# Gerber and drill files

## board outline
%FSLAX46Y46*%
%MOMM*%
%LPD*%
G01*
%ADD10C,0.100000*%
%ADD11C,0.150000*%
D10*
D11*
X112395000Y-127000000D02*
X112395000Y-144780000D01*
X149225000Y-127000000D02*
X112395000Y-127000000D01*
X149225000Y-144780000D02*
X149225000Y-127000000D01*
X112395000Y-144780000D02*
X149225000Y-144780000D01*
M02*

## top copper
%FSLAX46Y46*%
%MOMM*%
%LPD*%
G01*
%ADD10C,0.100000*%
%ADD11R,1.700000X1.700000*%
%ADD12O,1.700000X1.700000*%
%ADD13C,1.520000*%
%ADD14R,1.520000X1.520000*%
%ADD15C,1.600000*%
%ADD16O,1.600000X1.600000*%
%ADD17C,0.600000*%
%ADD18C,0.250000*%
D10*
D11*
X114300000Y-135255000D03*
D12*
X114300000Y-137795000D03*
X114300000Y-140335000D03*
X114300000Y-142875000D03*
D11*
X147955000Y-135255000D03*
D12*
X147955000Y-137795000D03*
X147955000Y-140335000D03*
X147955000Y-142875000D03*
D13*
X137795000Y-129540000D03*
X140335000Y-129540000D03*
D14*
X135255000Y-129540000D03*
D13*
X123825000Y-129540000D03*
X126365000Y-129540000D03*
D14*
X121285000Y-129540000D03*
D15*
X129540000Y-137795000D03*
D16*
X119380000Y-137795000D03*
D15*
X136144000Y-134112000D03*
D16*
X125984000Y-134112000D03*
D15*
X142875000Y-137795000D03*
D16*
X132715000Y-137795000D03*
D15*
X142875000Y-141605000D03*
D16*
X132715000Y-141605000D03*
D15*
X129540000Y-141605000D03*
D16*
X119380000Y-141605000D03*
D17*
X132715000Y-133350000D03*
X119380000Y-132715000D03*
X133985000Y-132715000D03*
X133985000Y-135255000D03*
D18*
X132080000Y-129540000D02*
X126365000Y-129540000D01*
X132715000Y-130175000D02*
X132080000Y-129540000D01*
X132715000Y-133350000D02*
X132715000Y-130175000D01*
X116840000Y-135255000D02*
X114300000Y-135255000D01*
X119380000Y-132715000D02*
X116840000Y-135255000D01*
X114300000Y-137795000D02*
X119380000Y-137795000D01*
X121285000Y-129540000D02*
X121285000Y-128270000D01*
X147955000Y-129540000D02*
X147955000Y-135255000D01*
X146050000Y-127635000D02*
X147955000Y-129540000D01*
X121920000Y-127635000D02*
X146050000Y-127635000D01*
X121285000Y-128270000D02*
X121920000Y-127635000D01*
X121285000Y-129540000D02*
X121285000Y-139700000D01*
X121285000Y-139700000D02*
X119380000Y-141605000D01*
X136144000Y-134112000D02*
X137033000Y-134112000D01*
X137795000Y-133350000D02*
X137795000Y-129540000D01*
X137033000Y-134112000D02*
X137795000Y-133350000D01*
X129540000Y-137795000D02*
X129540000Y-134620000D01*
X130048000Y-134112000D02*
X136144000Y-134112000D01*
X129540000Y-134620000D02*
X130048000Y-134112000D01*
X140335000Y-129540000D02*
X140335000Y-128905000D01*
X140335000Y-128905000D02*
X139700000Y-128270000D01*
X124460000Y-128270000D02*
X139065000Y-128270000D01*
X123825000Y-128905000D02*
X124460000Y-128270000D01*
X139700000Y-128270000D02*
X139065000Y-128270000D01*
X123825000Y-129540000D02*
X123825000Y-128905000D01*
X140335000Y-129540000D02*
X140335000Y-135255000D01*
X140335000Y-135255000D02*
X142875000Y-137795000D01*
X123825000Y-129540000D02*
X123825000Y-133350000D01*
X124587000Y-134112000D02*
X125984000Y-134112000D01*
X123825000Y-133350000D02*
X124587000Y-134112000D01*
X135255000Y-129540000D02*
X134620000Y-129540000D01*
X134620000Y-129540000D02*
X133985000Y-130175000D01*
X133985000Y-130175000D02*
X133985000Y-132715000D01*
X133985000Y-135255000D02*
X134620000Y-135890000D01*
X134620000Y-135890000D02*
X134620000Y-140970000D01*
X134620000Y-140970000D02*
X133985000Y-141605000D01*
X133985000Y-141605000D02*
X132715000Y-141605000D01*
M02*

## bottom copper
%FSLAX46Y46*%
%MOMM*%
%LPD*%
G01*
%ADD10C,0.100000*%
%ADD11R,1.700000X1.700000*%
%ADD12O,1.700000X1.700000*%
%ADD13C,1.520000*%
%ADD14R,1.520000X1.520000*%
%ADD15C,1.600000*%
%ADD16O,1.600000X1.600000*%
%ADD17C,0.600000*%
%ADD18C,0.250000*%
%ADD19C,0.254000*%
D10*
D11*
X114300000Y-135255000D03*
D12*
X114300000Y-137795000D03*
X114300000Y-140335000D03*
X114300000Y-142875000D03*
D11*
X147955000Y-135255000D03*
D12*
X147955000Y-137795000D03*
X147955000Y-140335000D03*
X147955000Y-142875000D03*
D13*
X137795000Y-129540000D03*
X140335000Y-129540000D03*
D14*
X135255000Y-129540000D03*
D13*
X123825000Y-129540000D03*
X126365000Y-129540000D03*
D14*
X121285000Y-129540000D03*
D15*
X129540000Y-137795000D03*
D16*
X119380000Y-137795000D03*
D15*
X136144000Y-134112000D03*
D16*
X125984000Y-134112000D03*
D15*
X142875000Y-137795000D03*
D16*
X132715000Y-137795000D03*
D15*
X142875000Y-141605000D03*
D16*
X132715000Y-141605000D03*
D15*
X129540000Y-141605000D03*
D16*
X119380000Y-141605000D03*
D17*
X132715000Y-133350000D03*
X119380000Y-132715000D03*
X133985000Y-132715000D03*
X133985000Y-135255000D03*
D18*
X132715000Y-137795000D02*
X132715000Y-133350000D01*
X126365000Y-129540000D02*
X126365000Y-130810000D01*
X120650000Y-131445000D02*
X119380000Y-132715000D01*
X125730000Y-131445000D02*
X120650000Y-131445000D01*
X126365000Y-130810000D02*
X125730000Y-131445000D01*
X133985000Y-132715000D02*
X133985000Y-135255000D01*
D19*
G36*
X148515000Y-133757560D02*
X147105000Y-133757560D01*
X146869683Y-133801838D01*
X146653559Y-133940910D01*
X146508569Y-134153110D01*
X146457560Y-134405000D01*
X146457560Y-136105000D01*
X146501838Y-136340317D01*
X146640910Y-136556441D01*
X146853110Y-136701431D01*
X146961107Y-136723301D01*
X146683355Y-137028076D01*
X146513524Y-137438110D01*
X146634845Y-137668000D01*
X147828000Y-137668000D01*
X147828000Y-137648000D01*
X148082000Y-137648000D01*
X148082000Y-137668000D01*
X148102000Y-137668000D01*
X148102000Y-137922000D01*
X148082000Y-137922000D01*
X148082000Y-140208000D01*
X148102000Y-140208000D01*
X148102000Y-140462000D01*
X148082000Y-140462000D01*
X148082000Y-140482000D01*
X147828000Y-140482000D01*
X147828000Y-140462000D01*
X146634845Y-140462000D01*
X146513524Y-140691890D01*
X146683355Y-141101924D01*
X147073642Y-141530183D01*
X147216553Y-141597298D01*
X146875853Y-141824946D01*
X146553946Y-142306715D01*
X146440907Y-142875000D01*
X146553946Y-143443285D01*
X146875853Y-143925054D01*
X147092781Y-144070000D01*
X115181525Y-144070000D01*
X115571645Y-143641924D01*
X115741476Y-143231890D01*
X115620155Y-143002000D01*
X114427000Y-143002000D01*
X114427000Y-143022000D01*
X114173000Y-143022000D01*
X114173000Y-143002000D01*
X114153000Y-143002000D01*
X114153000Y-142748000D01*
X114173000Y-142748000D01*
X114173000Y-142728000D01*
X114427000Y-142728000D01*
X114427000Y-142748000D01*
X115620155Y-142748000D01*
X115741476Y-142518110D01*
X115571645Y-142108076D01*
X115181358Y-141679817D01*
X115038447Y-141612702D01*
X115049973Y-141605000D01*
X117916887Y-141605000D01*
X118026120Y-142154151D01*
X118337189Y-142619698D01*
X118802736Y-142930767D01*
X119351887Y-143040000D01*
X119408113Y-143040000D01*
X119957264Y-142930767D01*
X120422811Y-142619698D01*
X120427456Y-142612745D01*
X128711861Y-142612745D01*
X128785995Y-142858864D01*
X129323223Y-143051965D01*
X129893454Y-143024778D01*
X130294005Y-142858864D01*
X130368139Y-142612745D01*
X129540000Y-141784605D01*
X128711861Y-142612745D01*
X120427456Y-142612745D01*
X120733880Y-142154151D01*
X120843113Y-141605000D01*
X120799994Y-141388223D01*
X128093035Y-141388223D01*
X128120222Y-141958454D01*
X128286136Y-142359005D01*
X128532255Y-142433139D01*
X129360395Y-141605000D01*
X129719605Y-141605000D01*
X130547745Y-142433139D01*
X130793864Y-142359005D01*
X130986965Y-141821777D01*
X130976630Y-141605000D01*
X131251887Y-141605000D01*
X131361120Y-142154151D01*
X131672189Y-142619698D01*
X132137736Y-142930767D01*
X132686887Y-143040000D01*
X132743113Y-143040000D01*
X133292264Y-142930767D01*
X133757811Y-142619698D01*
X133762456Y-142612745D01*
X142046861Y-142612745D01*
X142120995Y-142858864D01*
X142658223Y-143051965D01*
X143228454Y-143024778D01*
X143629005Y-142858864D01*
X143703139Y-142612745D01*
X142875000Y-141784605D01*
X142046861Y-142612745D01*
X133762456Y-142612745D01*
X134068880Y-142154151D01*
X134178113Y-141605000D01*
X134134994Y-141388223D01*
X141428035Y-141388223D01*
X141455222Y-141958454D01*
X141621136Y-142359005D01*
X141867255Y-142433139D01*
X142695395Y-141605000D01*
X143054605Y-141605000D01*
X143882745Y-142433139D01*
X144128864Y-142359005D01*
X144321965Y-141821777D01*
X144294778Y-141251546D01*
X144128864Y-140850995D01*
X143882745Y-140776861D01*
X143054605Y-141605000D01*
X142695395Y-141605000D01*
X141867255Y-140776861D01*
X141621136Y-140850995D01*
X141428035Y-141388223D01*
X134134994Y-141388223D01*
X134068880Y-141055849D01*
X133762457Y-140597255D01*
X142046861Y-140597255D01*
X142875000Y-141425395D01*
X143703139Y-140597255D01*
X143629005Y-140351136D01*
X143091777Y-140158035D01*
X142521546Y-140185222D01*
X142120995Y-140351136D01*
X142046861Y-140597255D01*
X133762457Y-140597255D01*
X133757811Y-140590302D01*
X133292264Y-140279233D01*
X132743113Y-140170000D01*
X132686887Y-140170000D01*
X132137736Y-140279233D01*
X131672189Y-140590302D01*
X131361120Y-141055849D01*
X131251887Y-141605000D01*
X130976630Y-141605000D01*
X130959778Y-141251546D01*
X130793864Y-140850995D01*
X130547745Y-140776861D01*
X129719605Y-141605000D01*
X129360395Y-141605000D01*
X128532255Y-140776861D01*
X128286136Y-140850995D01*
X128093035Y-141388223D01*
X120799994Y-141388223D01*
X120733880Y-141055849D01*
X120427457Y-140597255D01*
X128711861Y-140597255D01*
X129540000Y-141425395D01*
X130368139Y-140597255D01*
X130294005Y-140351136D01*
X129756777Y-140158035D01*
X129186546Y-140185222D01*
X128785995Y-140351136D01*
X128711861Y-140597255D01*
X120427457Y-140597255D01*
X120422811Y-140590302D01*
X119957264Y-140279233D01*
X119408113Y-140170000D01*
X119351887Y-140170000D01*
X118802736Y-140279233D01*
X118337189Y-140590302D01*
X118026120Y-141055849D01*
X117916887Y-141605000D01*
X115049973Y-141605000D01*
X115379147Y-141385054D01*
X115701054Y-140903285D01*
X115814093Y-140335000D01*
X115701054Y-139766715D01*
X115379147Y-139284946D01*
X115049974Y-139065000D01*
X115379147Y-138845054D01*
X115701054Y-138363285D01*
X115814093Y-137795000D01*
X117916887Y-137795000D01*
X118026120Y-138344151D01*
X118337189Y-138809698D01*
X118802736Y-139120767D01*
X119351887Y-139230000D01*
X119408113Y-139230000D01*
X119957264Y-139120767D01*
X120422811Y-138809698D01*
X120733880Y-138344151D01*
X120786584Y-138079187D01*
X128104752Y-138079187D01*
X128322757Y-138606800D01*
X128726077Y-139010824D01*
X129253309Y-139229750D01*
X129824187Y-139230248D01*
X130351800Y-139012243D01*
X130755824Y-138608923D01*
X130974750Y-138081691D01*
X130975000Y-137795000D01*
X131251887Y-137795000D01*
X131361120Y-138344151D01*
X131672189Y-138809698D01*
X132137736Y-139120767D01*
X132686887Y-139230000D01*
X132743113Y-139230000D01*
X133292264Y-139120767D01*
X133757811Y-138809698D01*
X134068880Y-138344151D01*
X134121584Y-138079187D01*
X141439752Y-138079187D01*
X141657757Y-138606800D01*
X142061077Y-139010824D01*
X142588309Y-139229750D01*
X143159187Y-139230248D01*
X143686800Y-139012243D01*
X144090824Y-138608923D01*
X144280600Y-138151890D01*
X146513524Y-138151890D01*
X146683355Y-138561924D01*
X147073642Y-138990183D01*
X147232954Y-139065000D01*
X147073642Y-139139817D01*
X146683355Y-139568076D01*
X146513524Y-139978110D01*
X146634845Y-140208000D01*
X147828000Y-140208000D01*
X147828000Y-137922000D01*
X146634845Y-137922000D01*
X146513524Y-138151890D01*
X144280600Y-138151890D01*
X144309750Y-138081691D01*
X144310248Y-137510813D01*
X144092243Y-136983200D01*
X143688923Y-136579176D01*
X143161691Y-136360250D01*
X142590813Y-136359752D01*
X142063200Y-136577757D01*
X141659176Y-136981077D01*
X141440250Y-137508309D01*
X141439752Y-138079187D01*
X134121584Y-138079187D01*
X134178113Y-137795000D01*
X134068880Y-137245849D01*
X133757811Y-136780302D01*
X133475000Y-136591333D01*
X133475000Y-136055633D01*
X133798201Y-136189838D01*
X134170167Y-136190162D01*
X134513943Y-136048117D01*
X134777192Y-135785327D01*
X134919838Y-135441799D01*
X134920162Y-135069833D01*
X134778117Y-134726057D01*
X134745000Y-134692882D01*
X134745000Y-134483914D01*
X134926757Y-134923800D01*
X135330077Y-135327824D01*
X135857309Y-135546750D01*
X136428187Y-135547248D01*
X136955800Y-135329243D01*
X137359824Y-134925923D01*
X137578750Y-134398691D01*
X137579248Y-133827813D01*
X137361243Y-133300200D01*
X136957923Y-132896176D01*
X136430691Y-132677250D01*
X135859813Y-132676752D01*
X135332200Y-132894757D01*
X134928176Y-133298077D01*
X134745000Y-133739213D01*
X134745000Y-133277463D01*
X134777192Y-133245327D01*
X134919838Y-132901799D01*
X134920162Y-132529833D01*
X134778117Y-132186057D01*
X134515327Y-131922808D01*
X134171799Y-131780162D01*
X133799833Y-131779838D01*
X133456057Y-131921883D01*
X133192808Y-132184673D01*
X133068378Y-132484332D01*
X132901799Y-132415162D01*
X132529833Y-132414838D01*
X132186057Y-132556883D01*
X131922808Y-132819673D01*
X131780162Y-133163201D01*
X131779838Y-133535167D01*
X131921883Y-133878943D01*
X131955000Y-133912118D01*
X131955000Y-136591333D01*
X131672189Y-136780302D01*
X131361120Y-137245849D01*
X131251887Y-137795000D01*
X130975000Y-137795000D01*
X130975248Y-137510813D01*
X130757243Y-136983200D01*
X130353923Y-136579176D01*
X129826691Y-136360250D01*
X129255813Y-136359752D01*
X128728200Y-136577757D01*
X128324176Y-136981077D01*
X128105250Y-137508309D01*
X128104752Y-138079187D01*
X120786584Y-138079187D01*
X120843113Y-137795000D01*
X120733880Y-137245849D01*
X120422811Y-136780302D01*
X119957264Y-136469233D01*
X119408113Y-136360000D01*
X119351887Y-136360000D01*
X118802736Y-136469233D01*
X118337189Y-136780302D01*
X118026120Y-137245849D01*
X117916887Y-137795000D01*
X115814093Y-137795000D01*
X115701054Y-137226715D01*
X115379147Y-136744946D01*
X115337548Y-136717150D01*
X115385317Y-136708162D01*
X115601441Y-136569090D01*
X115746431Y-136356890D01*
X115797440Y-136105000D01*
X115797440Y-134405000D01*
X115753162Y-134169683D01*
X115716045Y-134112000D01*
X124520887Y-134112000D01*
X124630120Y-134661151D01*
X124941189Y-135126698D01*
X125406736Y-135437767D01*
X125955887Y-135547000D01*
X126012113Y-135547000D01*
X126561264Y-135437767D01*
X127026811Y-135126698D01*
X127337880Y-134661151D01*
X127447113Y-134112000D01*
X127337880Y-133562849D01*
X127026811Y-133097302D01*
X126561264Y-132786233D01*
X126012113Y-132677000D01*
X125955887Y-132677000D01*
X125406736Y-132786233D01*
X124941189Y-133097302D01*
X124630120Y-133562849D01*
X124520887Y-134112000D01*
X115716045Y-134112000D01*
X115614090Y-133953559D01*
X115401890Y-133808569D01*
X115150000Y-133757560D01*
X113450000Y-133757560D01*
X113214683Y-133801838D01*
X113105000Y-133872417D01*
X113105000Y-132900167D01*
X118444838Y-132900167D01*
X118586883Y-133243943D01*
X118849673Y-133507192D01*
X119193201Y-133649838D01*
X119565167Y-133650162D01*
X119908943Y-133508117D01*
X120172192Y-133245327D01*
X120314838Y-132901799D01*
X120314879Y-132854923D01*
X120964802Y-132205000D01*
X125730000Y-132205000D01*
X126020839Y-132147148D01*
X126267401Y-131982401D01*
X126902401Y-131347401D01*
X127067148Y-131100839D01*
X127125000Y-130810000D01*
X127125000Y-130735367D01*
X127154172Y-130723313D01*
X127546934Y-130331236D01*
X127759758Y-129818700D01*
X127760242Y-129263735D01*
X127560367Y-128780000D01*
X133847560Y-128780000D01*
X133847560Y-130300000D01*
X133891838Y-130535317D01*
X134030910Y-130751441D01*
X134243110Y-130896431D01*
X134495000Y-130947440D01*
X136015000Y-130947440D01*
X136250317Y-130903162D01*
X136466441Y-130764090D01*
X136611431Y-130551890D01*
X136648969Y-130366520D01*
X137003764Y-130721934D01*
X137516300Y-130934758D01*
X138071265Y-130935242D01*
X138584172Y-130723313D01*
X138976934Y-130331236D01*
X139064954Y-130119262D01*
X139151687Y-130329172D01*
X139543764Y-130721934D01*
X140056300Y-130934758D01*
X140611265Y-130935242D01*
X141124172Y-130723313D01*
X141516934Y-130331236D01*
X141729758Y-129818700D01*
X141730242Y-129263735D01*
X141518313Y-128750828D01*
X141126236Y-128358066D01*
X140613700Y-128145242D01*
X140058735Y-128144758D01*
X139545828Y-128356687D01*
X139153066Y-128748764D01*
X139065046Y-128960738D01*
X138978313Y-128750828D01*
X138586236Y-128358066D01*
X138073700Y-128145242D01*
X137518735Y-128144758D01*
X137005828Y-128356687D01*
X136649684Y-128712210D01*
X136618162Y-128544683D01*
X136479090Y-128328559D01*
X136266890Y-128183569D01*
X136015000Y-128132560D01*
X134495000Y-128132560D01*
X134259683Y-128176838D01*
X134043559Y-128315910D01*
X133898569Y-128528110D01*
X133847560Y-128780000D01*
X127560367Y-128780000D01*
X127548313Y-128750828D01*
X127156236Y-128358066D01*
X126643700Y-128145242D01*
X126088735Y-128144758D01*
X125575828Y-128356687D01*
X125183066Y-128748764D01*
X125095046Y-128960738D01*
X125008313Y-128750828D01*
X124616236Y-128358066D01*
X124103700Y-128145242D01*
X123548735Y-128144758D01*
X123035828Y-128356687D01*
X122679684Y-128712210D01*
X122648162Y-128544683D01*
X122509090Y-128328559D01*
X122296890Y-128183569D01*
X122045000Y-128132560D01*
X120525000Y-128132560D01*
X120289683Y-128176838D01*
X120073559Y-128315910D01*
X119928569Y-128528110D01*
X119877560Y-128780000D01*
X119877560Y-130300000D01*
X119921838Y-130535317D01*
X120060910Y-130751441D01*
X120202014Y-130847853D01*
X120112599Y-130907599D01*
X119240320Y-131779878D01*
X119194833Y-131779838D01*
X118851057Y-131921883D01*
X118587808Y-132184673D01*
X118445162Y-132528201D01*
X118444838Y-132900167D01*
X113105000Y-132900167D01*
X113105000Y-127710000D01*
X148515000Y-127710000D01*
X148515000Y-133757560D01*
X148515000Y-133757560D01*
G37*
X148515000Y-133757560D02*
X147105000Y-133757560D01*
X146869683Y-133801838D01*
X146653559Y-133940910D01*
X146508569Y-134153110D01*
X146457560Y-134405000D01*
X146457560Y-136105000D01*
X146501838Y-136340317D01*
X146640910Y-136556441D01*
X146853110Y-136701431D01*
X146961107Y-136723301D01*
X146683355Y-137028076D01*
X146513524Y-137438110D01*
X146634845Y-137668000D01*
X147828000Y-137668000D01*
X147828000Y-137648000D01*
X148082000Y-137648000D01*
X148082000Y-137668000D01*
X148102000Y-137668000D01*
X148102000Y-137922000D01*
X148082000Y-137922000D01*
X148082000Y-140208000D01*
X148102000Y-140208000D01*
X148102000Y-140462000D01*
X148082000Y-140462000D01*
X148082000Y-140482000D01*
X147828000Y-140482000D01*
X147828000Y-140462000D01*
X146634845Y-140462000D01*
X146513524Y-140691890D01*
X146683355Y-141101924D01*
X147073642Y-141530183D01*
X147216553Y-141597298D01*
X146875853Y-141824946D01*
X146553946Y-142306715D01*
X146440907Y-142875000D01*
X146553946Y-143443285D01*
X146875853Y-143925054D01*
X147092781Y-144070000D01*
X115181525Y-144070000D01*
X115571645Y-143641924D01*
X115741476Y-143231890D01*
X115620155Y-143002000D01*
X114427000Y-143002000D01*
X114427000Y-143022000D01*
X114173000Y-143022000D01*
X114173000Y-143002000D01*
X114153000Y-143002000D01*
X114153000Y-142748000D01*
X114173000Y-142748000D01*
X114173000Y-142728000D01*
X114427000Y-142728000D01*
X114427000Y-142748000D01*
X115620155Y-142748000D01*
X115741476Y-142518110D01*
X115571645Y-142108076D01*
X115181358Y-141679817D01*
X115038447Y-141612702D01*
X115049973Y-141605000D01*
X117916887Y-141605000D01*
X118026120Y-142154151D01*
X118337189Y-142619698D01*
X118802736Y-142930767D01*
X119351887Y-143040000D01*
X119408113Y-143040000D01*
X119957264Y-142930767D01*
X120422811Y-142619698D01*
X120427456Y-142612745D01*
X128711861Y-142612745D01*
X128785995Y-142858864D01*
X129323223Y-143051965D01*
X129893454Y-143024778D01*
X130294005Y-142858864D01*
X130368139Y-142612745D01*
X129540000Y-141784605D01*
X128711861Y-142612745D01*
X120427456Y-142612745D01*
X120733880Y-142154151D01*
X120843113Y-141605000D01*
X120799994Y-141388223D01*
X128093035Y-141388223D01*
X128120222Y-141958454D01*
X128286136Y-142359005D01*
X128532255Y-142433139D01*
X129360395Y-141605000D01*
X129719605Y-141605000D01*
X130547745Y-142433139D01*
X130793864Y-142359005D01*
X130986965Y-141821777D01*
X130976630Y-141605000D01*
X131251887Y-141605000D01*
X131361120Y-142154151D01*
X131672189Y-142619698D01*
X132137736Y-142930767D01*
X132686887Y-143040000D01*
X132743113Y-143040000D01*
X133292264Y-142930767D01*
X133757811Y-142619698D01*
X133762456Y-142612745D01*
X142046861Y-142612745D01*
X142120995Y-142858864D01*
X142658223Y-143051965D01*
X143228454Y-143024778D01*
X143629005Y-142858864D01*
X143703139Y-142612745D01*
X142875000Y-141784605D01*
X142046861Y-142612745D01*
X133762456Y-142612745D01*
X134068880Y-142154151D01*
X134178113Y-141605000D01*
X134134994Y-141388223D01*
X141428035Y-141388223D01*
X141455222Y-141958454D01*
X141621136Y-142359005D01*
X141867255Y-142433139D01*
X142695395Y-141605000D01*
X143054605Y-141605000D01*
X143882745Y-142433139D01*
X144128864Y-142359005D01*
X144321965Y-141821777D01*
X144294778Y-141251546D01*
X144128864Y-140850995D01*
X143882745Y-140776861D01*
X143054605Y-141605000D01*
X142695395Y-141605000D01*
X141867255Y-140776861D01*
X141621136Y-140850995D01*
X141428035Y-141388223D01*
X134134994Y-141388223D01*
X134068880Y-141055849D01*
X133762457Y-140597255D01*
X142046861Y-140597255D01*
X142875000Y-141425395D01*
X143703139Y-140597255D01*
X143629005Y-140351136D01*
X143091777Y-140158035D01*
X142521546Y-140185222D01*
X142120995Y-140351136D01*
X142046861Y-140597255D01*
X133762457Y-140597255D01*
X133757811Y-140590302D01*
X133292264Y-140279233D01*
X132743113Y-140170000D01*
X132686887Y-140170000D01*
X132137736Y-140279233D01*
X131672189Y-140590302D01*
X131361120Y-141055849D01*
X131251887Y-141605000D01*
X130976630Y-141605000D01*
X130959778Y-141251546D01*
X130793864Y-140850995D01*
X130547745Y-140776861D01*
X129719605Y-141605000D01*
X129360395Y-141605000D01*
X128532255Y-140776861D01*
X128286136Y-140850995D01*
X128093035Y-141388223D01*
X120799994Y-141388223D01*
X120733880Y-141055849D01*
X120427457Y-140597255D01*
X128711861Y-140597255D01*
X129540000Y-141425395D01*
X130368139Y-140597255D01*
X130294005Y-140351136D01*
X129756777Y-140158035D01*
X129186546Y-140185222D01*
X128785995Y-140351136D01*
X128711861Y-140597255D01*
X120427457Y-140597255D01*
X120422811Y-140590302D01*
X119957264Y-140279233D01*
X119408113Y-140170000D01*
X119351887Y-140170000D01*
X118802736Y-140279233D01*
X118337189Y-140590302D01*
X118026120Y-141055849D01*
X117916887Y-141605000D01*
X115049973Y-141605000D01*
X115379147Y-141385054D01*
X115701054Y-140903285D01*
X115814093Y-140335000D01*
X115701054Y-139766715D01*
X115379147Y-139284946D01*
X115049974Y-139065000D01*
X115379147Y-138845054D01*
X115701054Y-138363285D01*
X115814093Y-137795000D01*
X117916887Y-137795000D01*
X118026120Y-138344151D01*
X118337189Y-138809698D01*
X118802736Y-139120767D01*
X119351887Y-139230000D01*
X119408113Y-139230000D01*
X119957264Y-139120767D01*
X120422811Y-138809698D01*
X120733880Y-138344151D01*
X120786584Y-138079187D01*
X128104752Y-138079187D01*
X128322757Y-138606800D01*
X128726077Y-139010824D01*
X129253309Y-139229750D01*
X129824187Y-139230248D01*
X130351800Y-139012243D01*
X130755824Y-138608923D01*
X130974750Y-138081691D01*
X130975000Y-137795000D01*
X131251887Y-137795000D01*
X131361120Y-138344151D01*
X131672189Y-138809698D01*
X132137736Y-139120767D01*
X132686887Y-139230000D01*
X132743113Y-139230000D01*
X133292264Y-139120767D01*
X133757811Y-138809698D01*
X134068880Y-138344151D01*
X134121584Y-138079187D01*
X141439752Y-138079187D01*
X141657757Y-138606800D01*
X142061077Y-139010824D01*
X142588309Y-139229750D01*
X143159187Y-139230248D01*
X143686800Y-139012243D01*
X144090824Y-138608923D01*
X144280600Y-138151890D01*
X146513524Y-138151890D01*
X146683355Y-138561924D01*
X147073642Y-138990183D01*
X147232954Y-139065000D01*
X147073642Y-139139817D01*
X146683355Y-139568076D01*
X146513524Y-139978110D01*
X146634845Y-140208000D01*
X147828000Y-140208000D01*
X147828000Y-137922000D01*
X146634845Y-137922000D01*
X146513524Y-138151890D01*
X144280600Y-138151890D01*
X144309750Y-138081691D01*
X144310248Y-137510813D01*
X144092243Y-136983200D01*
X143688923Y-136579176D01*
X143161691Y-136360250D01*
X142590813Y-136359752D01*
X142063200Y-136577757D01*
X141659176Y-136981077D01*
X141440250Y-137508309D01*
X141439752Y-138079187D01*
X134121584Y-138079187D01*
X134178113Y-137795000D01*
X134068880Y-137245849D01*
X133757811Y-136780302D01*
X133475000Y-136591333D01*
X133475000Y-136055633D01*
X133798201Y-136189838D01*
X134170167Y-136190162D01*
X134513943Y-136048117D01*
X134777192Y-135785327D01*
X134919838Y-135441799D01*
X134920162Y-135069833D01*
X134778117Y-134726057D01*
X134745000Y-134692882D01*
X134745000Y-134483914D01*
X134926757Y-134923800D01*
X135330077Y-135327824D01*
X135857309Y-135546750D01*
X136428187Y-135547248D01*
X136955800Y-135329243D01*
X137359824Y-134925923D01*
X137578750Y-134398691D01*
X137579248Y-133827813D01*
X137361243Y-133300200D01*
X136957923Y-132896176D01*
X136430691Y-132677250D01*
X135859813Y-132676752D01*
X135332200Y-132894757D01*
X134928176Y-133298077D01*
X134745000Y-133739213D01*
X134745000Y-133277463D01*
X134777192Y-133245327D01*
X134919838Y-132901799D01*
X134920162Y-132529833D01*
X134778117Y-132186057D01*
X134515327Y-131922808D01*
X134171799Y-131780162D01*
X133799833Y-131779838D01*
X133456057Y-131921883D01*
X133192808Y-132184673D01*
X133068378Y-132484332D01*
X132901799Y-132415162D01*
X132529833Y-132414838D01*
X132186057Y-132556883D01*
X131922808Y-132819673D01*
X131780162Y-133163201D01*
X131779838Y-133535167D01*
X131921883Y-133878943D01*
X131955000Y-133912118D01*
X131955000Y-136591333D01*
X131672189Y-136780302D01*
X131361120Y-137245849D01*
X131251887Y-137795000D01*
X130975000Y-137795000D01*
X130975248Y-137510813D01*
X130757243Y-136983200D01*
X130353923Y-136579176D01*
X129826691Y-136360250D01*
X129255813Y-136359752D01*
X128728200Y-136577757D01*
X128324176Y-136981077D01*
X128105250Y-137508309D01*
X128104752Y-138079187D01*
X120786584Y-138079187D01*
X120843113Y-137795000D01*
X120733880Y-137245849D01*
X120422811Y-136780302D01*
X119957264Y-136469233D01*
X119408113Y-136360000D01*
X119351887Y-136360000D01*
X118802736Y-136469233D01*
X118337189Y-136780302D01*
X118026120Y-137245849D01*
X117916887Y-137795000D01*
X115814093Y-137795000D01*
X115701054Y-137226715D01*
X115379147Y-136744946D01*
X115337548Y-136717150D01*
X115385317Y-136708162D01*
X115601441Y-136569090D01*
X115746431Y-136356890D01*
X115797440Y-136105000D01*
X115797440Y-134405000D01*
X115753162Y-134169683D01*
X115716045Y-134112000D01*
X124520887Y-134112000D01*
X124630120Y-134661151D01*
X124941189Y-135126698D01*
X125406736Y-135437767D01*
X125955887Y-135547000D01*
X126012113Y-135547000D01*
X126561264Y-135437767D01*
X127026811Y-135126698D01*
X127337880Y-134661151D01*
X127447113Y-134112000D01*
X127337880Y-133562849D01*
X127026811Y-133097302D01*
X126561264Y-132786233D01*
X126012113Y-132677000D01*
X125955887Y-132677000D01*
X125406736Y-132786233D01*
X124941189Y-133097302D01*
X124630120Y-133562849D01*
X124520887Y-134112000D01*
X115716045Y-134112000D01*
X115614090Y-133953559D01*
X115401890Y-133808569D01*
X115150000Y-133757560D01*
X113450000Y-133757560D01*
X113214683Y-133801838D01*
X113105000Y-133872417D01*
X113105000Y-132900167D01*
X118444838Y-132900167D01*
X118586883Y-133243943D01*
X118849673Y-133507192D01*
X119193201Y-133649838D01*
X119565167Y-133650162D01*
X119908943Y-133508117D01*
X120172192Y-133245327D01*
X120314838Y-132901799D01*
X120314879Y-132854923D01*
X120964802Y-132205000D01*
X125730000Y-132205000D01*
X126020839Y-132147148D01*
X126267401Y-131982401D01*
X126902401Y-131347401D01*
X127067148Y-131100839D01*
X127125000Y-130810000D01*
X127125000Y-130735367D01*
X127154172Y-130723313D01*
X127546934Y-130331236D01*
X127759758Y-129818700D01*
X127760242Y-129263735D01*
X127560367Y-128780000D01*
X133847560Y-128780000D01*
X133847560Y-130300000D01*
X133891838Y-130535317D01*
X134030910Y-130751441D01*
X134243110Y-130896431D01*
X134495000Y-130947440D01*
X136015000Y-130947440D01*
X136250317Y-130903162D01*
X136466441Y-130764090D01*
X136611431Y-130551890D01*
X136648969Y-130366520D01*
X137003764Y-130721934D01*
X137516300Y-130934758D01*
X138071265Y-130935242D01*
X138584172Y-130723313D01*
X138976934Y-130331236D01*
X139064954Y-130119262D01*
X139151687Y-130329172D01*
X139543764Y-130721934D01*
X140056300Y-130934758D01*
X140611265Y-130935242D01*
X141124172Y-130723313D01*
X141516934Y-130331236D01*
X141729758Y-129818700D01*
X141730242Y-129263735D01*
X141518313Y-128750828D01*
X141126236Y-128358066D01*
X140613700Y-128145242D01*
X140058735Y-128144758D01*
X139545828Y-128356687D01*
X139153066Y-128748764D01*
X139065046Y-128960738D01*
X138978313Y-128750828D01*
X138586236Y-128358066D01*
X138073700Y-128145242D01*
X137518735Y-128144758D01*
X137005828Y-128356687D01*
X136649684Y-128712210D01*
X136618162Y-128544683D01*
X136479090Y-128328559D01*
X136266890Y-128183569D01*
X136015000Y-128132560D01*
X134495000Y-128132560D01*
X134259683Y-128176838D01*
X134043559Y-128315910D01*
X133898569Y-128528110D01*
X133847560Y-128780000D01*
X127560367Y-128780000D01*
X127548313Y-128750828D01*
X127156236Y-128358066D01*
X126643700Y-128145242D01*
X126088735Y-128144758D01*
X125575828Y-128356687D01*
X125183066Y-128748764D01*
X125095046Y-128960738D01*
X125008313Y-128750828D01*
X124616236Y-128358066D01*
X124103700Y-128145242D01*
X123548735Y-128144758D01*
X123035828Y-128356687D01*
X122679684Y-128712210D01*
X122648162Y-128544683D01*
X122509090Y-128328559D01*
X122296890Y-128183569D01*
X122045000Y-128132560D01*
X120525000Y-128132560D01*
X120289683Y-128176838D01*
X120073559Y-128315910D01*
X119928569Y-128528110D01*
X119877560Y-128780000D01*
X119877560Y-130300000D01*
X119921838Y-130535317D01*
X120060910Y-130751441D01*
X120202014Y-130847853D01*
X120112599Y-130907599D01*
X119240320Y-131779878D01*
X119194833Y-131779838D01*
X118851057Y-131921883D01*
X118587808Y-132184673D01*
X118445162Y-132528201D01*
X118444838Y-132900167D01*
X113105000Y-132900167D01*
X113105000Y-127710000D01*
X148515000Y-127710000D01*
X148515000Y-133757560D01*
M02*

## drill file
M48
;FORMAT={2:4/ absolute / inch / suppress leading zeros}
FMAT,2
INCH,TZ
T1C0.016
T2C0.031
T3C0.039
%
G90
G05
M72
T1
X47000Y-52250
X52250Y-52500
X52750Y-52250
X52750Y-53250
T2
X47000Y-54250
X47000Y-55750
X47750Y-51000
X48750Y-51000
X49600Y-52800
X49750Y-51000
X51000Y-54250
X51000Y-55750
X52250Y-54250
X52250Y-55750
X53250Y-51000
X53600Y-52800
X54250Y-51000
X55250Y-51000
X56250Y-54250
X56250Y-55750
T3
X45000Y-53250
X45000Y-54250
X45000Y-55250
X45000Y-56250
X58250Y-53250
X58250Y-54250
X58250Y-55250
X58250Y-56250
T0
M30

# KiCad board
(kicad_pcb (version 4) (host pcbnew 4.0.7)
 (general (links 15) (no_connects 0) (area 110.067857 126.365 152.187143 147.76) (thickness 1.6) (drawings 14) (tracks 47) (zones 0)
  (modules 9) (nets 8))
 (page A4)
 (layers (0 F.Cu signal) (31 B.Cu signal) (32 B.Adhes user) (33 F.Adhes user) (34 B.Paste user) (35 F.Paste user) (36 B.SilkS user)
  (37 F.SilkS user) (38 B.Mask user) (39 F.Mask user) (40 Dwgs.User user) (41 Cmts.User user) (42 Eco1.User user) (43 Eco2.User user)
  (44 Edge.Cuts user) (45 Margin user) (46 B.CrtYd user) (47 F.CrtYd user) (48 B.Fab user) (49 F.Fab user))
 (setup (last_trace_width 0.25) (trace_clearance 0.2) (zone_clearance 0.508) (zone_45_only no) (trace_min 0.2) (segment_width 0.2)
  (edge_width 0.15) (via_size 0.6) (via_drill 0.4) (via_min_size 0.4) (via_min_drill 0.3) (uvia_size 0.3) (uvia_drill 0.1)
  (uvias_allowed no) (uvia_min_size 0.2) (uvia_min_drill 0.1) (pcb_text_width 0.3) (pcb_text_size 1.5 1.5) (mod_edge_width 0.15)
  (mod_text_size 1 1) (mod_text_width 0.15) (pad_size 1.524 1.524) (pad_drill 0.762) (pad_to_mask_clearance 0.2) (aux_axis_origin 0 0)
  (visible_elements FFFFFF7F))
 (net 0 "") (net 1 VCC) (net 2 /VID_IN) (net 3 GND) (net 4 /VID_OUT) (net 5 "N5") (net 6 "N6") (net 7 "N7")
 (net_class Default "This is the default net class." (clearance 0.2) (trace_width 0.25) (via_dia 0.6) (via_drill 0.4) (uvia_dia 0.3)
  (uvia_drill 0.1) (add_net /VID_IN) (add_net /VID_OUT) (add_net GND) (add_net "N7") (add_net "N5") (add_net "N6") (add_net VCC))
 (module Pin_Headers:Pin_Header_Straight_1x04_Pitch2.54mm (layer F.Cu) (at 114.3 135.255)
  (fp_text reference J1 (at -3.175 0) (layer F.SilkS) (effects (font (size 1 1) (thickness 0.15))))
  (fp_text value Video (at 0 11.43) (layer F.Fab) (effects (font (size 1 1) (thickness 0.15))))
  (pad 1 thru_hole rect (at 0 0) (size 1.7 1.7) (drill 1) (layers *.Cu *.Mask) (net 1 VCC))
  (pad 2 thru_hole oval (at 0 2.54) (size 1.7 1.7) (drill 1) (layers *.Cu *.Mask) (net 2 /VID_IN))
  (pad 3 thru_hole oval (at 0 5.08) (size 1.7 1.7) (drill 1) (layers *.Cu *.Mask))
  (pad 4 thru_hole oval (at 0 7.62) (size 1.7 1.7) (drill 1) (layers *.Cu *.Mask) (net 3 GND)))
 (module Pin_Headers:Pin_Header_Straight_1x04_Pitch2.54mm (layer F.Cu) (at 147.955 135.255)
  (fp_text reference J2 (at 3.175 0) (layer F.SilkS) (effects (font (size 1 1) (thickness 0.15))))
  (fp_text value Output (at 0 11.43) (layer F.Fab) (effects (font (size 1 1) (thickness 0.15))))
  (pad 1 thru_hole rect (at 0 0) (size 1.7 1.7) (drill 1) (layers *.Cu *.Mask) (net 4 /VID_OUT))
  (pad 2 thru_hole oval (at 0 2.54) (size 1.7 1.7) (drill 1) (layers *.Cu *.Mask) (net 3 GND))
  (pad 3 thru_hole oval (at 0 5.08) (size 1.7 1.7) (drill 1) (layers *.Cu *.Mask) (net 3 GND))
  (pad 4 thru_hole oval (at 0 7.62) (size 1.7 1.7) (drill 1) (layers *.Cu *.Mask)))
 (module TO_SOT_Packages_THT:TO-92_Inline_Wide (layer F.Cu) (at 135.255 129.54)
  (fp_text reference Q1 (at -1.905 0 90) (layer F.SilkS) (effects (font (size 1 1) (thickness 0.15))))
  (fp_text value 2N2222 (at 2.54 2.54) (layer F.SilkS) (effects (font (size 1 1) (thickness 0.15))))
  (pad 2 thru_hole circle (at 2.54 0 90) (size 1.52 1.52) (drill 0.8) (layers *.Cu *.Mask) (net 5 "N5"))
  (pad 3 thru_hole circle (at 5.08 0 90) (size 1.52 1.52) (drill 0.8) (layers *.Cu *.Mask) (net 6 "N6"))
  (pad 1 thru_hole rect (at 0 0 90) (size 1.52 1.52) (drill 0.8) (layers *.Cu *.Mask) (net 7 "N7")))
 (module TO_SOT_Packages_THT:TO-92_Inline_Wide (layer F.Cu) (at 121.285 129.54)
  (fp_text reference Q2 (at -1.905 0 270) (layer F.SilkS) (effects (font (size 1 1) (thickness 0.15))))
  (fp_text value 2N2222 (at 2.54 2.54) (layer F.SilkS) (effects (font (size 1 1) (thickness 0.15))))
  (pad 2 thru_hole circle (at 2.54 0 90) (size 1.52 1.52) (drill 0.8) (layers *.Cu *.Mask) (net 6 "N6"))
  (pad 3 thru_hole circle (at 5.08 0 90) (size 1.52 1.52) (drill 0.8) (layers *.Cu *.Mask) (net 1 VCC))
  (pad 1 thru_hole rect (at 0 0 90) (size 1.52 1.52) (drill 0.8) (layers *.Cu *.Mask) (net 4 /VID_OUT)))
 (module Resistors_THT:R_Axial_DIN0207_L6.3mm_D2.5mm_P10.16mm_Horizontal (layer F.Cu) (at 129.54 137.795 180)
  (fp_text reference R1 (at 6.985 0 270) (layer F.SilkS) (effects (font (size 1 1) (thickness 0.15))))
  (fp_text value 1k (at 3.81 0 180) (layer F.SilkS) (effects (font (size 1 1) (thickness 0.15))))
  (pad 1 thru_hole circle (at 0 0 180) (size 1.6 1.6) (drill 0.8) (layers *.Cu *.Mask) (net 5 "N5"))
  (pad 2 thru_hole oval (at 10.16 0 180) (size 1.6 1.6) (drill 0.8) (layers *.Cu *.Mask) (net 2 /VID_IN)))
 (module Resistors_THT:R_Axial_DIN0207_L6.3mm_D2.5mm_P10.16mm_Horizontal (layer F.Cu) (at 136.144 134.112 180)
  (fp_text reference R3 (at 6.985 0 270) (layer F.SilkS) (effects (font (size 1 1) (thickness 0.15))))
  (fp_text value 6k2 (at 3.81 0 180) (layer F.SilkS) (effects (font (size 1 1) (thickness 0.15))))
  (pad 1 thru_hole circle (at 0 0 180) (size 1.6 1.6) (drill 0.8) (layers *.Cu *.Mask) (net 5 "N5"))
  (pad 2 thru_hole oval (at 10.16 0 180) (size 1.6 1.6) (drill 0.8) (layers *.Cu *.Mask) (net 6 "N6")))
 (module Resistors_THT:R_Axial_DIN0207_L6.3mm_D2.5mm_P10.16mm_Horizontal (layer F.Cu) (at 142.875 137.795 180)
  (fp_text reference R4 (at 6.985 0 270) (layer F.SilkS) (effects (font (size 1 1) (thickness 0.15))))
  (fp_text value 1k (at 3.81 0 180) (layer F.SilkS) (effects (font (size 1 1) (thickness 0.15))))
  (pad 1 thru_hole circle (at 0 0 180) (size 1.6 1.6) (drill 0.8) (layers *.Cu *.Mask) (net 6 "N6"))
  (pad 2 thru_hole oval (at 10.16 0 180) (size 1.6 1.6) (drill 0.8) (layers *.Cu *.Mask) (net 1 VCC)))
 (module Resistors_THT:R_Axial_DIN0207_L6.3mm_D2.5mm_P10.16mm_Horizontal (layer F.Cu) (at 142.875 141.605 180)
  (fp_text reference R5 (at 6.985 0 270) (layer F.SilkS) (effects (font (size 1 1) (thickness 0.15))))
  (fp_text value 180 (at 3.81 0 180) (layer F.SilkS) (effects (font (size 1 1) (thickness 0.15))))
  (pad 1 thru_hole circle (at 0 0 180) (size 1.6 1.6) (drill 0.8) (layers *.Cu *.Mask) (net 3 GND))
  (pad 2 thru_hole oval (at 10.16 0 180) (size 1.6 1.6) (drill 0.8) (layers *.Cu *.Mask) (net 7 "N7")))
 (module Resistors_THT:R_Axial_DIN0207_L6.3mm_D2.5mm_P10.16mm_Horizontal (layer F.Cu) (at 129.54 141.605 180)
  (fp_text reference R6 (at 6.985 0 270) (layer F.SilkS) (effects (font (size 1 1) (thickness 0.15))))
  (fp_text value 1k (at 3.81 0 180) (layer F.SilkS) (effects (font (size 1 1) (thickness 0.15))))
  (pad 1 thru_hole circle (at 0 0 180) (size 1.6 1.6) (drill 0.8) (layers *.Cu *.Mask) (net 3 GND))
  (pad 2 thru_hole oval (at 10.16 0 180) (size 1.6 1.6) (drill 0.8) (layers *.Cu *.Mask) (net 4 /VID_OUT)))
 (gr_line (start 112.395 127) (end 112.395 144.78) (angle 90) (layer Edge.Cuts) (width 0.15))
 (gr_line (start 149.225 127) (end 112.395 127) (angle 90) (layer Edge.Cuts) (width 0.15))
 (gr_line (start 149.225 144.78) (end 149.225 127) (angle 90) (layer Edge.Cuts) (width 0.15))
 (gr_line (start 112.395 144.78) (end 149.225 144.78) (angle 90) (layer Edge.Cuts) (width 0.15))
 (segment (start 132.715 137.795) (end 132.715 133.35) (width 0.25) (layer B.Cu) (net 1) (status 400000))
 (segment (start 132.08 129.54) (end 126.365 129.54) (width 0.25) (layer F.Cu) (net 1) (status 800000))
 (segment (start 132.715 130.175) (end 132.08 129.54) (width 0.25) (layer F.Cu) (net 1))
 (segment (start 132.715 133.35) (end 132.715 130.175) (width 0.25) (layer F.Cu) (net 1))
 (via (at 132.715 133.35) (size 0.6) (drill 0.4) (layers F.Cu B.Cu) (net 1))
 (segment (start 126.365 129.54) (end 126.365 130.81) (width 0.25) (layer B.Cu) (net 1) (status 400000))
 (segment (start 116.84 135.255) (end 114.3 135.255) (width 0.25) (layer F.Cu) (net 1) (status 800000))
 (segment (start 119.38 132.715) (end 116.84 135.255) (width 0.25) (layer F.Cu) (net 1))
 (via (at 119.38 132.715) (size 0.6) (drill 0.4) (layers F.Cu B.Cu) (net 1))
 (segment (start 120.65 131.445) (end 119.38 132.715) (width 0.25) (layer B.Cu) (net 1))
 (segment (start 125.73 131.445) (end 120.65 131.445) (width 0.25) (layer B.Cu) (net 1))
 (segment (start 126.365 130.81) (end 125.73 131.445) (width 0.25) (layer B.Cu) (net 1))
 (segment (start 114.3 137.795) (end 119.38 137.795) (width 0.25) (layer F.Cu) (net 2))
 (segment (start 121.285 129.54) (end 121.285 128.27) (width 0.25) (layer F.Cu) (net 4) (status 400000))
 (segment (start 147.955 129.54) (end 147.955 135.255) (width 0.25) (layer F.Cu) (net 4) (status 800000))
 (segment (start 146.05 127.635) (end 147.955 129.54) (width 0.25) (layer F.Cu) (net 4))
 (segment (start 121.92 127.635) (end 146.05 127.635) (width 0.25) (layer F.Cu) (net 4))
 (segment (start 121.285 128.27) (end 121.92 127.635) (width 0.25) (layer F.Cu) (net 4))
 (segment (start 121.285 129.54) (end 121.285 139.7) (width 0.25) (layer F.Cu) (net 4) (status 400000))
 (segment (start 121.285 139.7) (end 119.38 141.605) (width 0.25) (layer F.Cu) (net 4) (status 800000))
 (segment (start 136.144 134.112) (end 137.033 134.112) (width 0.25) (layer F.Cu) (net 5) (status 400000))
 (segment (start 137.795 133.35) (end 137.795 129.54) (width 0.25) (layer F.Cu) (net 5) (status 800000))
 (segment (start 137.033 134.112) (end 137.795 133.35) (width 0.25) (layer F.Cu) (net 5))
 (segment (start 129.54 137.795) (end 129.54 134.62) (width 0.25) (layer F.Cu) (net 5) (status 400000))
 (segment (start 130.048 134.112) (end 136.144 134.112) (width 0.25) (layer F.Cu) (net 5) (status 800000))
 (segment (start 129.54 134.62) (end 130.048 134.112) (width 0.25) (layer F.Cu) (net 5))
 (segment (start 140.335 129.54) (end 140.335 128.905) (width 0.25) (layer F.Cu) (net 6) (status C00000))
 (segment (start 140.335 128.905) (end 139.7 128.27) (width 0.25) (layer F.Cu) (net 6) (status 400000))
 (segment (start 124.46 128.27) (end 139.065 128.27) (width 0.25) (layer F.Cu) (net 6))
 (segment (start 123.825 128.905) (end 124.46 128.27) (width 0.25) (layer F.Cu) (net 6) (status 400000))
 (segment (start 139.7 128.27) (end 139.065 128.27) (width 0.25) (layer F.Cu) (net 6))
 (segment (start 123.825 129.54) (end 123.825 128.905) (width 0.25) (layer F.Cu) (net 6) (status C00000))
 (segment (start 140.335 129.54) (end 140.335 135.255) (width 0.25) (layer F.Cu) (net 6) (status 400000))
 (segment (start 140.335 135.255) (end 142.875 137.795) (width 0.25) (layer F.Cu) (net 6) (status 800000))
 (segment (start 123.825 129.54) (end 123.825 133.35) (width 0.25) (layer F.Cu) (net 6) (status 400000))
 (segment (start 124.587 134.112) (end 125.984 134.112) (width 0.25) (layer F.Cu) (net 6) (status 800000))
 (segment (start 123.825 133.35) (end 124.587 134.112) (width 0.25) (layer F.Cu) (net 6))
 (segment (start 135.255 129.54) (end 134.62 129.54) (width 0.25) (layer F.Cu) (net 7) (status C00000))
 (segment (start 134.62 129.54) (end 133.985 130.175) (width 0.25) (layer F.Cu) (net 7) (status 400000))
 (segment (start 133.985 130.175) (end 133.985 132.715) (width 0.25) (layer F.Cu) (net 7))
 (via (at 133.985 132.715) (size 0.6) (drill 0.4) (layers F.Cu B.Cu) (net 7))
 (segment (start 133.985 132.715) (end 133.985 135.255) (width 0.25) (layer B.Cu) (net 7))
 (via (at 133.985 135.255) (size 0.6) (drill 0.4) (layers F.Cu B.Cu) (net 7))
 (segment (start 133.985 135.255) (end 134.62 135.89) (width 0.25) (layer F.Cu) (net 7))
 (segment (start 134.62 135.89) (end 134.62 140.97) (width 0.25) (layer F.Cu) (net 7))
 (segment (start 134.62 140.97) (end 133.985 141.605) (width 0.25) (layer F.Cu) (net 7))
 (segment (start 133.985 141.605) (end 132.715 141.605) (width 0.25) (layer F.Cu) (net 7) (status 800000))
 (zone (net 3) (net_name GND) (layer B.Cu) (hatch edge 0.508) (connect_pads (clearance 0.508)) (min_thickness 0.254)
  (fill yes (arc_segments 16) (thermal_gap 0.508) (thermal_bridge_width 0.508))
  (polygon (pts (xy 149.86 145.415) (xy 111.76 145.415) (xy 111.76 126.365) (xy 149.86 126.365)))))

